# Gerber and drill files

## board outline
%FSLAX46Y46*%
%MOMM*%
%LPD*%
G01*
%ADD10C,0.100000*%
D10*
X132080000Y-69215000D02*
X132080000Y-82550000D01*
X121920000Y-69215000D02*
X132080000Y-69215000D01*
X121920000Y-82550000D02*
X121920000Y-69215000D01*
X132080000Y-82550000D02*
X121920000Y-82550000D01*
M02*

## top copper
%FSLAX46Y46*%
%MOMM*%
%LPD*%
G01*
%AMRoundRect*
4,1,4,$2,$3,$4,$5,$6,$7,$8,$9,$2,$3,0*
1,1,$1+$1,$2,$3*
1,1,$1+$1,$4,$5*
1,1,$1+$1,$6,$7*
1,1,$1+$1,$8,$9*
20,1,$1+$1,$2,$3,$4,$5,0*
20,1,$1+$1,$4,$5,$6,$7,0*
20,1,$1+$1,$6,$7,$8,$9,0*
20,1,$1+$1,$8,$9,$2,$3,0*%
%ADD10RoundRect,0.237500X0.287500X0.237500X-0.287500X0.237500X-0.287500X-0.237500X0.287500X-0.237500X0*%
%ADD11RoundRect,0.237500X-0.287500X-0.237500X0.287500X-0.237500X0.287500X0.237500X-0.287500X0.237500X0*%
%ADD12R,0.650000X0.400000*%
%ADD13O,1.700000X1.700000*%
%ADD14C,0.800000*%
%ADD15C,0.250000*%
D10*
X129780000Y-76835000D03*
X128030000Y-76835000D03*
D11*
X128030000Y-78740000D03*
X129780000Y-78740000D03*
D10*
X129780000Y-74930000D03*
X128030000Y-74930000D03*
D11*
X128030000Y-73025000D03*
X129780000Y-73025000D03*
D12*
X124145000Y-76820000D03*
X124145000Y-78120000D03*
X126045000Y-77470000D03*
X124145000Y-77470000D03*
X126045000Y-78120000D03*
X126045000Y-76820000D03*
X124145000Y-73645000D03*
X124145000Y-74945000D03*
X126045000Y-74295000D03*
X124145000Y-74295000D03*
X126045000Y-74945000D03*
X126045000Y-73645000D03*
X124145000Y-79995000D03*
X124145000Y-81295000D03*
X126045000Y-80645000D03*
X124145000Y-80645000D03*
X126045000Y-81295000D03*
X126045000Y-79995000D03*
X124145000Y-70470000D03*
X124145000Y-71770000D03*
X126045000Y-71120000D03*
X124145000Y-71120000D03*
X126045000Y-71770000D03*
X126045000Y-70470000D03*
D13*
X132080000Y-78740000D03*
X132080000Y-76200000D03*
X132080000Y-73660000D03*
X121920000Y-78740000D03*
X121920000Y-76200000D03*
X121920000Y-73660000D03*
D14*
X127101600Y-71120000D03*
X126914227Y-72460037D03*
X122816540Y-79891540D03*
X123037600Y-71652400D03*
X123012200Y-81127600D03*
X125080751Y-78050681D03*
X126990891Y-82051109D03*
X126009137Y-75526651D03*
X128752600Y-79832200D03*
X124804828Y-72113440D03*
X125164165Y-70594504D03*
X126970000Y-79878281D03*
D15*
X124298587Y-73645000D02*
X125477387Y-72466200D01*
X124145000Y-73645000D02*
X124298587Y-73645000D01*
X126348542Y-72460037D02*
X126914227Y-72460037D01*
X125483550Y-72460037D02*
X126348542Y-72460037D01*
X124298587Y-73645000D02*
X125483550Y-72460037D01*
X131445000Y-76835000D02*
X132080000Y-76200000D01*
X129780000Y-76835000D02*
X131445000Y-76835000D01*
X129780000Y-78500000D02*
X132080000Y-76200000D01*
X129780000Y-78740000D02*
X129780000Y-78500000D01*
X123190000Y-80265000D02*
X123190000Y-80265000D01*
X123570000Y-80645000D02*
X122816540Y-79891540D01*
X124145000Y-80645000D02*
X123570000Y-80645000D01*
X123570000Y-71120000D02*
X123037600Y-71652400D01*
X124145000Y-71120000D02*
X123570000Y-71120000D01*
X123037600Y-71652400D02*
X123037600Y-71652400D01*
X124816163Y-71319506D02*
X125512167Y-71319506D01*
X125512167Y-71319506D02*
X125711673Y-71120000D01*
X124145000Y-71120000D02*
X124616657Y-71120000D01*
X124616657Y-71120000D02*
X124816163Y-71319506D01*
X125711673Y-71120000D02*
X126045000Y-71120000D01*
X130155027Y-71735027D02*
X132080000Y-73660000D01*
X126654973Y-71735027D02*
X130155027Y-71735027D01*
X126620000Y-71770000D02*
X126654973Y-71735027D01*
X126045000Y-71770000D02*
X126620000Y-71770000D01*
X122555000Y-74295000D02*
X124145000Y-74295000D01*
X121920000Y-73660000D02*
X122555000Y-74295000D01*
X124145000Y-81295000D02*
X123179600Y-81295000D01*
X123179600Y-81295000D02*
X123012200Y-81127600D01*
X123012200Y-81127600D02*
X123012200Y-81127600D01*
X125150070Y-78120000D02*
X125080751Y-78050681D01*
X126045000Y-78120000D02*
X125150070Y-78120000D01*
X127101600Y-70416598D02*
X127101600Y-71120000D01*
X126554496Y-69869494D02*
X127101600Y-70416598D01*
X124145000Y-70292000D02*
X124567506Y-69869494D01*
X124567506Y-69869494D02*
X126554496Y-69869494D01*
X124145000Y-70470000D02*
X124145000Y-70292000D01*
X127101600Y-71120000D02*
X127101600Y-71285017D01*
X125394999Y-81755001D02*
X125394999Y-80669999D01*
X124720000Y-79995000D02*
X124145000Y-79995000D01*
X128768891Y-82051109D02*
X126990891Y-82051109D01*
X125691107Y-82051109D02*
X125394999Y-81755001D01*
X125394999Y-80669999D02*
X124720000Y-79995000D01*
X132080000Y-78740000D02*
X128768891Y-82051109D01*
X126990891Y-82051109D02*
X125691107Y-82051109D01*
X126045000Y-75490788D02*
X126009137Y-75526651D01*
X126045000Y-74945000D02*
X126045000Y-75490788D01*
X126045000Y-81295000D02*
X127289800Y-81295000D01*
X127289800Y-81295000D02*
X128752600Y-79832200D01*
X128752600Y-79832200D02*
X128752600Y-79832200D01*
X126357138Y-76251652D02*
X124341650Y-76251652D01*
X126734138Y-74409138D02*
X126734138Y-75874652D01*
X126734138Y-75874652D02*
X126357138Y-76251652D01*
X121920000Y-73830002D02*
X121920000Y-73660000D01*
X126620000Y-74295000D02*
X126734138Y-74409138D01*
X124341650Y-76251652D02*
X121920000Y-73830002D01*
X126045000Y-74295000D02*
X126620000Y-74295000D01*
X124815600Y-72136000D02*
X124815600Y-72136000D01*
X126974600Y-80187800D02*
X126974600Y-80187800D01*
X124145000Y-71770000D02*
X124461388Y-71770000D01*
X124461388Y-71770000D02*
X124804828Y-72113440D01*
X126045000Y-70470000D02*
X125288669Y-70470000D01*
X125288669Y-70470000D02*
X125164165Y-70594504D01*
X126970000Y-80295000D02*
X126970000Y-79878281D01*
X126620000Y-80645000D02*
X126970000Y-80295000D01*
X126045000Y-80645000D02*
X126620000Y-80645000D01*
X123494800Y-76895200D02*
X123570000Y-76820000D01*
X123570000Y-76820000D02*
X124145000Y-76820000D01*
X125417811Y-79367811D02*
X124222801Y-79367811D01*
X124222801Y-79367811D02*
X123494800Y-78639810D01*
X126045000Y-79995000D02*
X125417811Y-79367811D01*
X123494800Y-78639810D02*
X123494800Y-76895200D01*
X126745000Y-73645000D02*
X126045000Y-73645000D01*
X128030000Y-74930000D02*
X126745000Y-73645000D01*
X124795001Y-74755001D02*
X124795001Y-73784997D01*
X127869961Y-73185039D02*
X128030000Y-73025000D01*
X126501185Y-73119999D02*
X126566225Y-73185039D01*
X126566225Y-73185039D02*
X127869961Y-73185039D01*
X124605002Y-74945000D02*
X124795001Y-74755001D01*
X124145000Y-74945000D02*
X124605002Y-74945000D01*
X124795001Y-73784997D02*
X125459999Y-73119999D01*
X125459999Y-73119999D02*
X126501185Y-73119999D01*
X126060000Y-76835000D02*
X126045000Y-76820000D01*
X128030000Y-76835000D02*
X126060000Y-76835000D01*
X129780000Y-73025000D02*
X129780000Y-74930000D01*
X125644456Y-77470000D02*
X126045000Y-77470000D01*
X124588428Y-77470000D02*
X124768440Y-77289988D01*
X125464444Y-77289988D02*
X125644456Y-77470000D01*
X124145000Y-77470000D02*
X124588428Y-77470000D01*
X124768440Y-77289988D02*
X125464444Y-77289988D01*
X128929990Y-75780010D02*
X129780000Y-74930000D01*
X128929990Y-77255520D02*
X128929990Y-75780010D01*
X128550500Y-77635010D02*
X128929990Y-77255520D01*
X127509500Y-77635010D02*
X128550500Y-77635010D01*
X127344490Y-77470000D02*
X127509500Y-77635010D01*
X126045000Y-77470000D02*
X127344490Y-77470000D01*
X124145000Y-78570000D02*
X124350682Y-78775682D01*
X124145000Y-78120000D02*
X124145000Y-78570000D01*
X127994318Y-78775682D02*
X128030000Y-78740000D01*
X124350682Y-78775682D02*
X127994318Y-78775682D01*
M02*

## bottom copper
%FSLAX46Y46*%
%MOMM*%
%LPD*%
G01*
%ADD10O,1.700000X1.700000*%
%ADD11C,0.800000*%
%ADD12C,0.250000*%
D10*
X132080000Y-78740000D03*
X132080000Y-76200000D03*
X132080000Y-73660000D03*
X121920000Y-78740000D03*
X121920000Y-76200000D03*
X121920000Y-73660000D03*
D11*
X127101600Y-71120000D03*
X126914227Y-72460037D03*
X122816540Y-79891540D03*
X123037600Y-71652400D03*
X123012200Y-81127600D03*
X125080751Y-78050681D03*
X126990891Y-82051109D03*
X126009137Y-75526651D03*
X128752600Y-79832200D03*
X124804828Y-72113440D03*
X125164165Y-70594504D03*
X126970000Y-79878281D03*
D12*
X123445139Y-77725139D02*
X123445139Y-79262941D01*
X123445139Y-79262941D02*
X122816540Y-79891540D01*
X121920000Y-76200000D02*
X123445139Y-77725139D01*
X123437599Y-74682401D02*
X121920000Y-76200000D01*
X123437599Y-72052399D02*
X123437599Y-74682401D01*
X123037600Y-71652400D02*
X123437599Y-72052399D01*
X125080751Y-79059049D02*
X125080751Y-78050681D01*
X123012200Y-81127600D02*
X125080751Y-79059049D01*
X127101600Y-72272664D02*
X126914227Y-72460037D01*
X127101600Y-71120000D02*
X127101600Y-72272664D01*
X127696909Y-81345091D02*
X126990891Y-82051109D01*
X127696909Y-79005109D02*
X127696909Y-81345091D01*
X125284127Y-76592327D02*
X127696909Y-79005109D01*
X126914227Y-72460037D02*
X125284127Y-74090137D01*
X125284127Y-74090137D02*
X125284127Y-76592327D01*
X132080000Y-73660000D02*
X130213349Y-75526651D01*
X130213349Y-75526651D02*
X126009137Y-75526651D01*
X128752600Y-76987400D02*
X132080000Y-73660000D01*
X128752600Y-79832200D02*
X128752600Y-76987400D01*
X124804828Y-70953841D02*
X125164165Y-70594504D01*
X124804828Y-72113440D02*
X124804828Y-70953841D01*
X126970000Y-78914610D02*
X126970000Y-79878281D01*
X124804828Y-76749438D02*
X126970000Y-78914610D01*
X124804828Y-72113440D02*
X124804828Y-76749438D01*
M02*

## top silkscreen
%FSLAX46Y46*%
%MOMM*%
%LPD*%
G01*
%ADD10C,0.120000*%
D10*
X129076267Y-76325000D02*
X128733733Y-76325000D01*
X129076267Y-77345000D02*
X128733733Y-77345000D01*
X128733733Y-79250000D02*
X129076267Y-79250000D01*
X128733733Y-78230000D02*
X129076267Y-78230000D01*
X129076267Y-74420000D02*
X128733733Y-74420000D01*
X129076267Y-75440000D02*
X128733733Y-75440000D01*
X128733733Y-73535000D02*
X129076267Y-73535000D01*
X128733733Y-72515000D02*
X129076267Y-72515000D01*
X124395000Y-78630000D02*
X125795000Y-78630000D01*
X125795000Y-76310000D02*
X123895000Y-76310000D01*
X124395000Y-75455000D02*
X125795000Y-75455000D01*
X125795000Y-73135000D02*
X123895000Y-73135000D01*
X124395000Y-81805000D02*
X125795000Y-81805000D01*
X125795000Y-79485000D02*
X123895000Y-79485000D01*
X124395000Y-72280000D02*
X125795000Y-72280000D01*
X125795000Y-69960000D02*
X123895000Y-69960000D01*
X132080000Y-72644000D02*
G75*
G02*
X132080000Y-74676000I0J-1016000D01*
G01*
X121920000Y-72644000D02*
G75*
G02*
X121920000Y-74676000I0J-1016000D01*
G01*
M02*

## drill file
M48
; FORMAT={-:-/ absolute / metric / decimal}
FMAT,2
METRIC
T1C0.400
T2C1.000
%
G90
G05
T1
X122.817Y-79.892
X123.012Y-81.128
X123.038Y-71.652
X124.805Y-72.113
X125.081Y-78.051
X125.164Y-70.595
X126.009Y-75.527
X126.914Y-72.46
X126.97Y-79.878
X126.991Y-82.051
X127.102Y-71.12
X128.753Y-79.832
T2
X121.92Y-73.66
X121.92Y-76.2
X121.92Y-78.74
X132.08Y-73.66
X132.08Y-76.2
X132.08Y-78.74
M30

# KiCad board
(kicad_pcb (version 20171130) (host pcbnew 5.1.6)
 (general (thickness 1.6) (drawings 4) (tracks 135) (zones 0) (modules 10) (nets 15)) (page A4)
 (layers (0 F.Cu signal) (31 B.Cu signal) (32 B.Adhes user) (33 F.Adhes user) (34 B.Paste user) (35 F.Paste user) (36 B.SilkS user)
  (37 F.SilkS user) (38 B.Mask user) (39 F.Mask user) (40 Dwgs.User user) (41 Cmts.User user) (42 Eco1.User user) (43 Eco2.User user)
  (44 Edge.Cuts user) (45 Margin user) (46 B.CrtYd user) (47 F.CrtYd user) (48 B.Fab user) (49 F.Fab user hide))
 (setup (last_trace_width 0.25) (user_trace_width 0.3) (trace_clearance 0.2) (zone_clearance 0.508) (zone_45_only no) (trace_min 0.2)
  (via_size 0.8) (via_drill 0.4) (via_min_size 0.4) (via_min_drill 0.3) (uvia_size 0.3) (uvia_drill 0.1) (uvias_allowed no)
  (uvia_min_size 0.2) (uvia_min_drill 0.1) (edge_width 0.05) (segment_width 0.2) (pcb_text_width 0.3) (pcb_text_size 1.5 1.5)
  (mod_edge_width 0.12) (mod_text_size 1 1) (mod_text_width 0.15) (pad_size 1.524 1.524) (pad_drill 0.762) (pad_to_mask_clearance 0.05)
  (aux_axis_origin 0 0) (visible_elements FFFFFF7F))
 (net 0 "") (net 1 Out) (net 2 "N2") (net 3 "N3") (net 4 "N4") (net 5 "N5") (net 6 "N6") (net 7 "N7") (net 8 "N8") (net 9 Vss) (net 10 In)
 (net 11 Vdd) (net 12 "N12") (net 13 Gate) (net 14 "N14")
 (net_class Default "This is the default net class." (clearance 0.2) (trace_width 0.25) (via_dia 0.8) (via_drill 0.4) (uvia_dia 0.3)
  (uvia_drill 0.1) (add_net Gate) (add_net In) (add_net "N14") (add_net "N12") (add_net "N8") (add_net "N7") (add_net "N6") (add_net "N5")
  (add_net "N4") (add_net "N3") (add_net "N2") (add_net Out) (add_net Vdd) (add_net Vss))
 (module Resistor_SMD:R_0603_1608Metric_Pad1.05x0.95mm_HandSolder (layer F.Cu) (at 128.905 76.835 180)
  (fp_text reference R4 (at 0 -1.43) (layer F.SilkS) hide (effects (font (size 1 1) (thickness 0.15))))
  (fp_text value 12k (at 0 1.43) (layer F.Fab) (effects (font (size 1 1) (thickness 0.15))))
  (fp_line (start -0.171267 0.51) (end 0.171267 0.51) (layer F.SilkS) (width 0.12))
  (fp_line (start -0.171267 -0.51) (end 0.171267 -0.51) (layer F.SilkS) (width 0.12))
  (pad 1 smd roundrect (at -0.875 0 180) (size 1.05 0.95) (layers F.Cu F.Paste F.Mask) (roundrect_rratio 0.25) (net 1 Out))
  (pad 2 smd roundrect (at 0.875 0 180) (size 1.05 0.95) (layers F.Cu F.Paste F.Mask) (roundrect_rratio 0.25) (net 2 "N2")))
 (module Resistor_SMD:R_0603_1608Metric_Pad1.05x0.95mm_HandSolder (layer F.Cu) (at 128.905 78.74)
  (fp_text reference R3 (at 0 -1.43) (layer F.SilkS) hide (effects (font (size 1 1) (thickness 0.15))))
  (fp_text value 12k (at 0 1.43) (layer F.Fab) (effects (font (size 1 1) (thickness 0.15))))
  (fp_line (start -0.171267 0.51) (end 0.171267 0.51) (layer F.SilkS) (width 0.12))
  (fp_line (start -0.171267 -0.51) (end 0.171267 -0.51) (layer F.SilkS) (width 0.12))
  (pad 1 smd roundrect (at -0.875 0) (size 1.05 0.95) (layers F.Cu F.Paste F.Mask) (roundrect_rratio 0.25) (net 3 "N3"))
  (pad 2 smd roundrect (at 0.875 0) (size 1.05 0.95) (layers F.Cu F.Paste F.Mask) (roundrect_rratio 0.25) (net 1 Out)))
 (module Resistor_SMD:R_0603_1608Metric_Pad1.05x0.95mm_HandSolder (layer F.Cu) (at 128.905 74.93 180)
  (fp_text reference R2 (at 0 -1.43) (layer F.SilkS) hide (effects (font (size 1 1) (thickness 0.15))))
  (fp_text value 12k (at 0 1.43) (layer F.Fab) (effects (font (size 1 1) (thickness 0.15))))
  (fp_line (start -0.171267 0.51) (end 0.171267 0.51) (layer F.SilkS) (width 0.12))
  (fp_line (start -0.171267 -0.51) (end 0.171267 -0.51) (layer F.SilkS) (width 0.12))
  (pad 1 smd roundrect (at -0.875 0 180) (size 1.05 0.95) (layers F.Cu F.Paste F.Mask) (roundrect_rratio 0.25) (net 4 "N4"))
  (pad 2 smd roundrect (at 0.875 0 180) (size 1.05 0.95) (layers F.Cu F.Paste F.Mask) (roundrect_rratio 0.25) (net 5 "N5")))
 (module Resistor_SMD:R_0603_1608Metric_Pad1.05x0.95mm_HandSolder (layer F.Cu) (at 128.905 73.025)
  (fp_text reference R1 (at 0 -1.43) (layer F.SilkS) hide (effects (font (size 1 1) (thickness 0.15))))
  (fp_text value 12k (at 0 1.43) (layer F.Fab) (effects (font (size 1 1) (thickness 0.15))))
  (fp_line (start -0.171267 0.51) (end 0.171267 0.51) (layer F.SilkS) (width 0.12))
  (fp_line (start -0.171267 -0.51) (end 0.171267 -0.51) (layer F.SilkS) (width 0.12))
  (pad 1 smd roundrect (at -0.875 0) (size 1.05 0.95) (layers F.Cu F.Paste F.Mask) (roundrect_rratio 0.25) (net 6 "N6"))
  (pad 2 smd roundrect (at 0.875 0) (size 1.05 0.95) (layers F.Cu F.Paste F.Mask) (roundrect_rratio 0.25) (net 4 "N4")))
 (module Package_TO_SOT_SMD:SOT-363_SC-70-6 (layer F.Cu) (at 125.095 77.47)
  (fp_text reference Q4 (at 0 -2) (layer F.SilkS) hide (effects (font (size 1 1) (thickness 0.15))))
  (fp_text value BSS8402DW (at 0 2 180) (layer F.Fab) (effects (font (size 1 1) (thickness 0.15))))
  (fp_line (start -0.7 1.16) (end 0.7 1.16) (layer F.SilkS) (width 0.12))
  (fp_line (start 0.7 -1.16) (end -1.2 -1.16) (layer F.SilkS) (width 0.12))
  (pad 1 smd rect (at -0.95 -0.65) (size 0.65 0.4) (layers F.Cu F.Paste F.Mask) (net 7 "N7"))
  (pad 3 smd rect (at -0.95 0.65) (size 0.65 0.4) (layers F.Cu F.Paste F.Mask) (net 3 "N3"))
  (pad 5 smd rect (at 0.95 0) (size 0.65 0.4) (layers F.Cu F.Paste F.Mask) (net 4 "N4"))
  (pad 2 smd rect (at -0.95 0) (size 0.65 0.4) (layers F.Cu F.Paste F.Mask) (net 4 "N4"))
  (pad 4 smd rect (at 0.95 0.65) (size 0.65 0.4) (layers F.Cu F.Paste F.Mask) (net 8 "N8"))
  (pad 6 smd rect (at 0.95 -0.65) (size 0.65 0.4) (layers F.Cu F.Paste F.Mask) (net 2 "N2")))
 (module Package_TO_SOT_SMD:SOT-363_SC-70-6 (layer F.Cu) (at 125.095 74.295)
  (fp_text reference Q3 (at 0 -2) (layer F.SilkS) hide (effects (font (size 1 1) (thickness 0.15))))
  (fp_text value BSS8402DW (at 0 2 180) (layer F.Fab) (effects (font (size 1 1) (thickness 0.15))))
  (fp_line (start -0.7 1.16) (end 0.7 1.16) (layer F.SilkS) (width 0.12))
  (fp_line (start 0.7 -1.16) (end -1.2 -1.16) (layer F.SilkS) (width 0.12))
  (pad 1 smd rect (at -0.95 -0.65) (size 0.65 0.4) (layers F.Cu F.Paste F.Mask) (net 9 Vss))
  (pad 3 smd rect (at -0.95 0.65) (size 0.65 0.4) (layers F.Cu F.Paste F.Mask) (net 6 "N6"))
  (pad 5 smd rect (at 0.95 0) (size 0.65 0.4) (layers F.Cu F.Paste F.Mask) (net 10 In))
  (pad 2 smd rect (at -0.95 0) (size 0.65 0.4) (layers F.Cu F.Paste F.Mask) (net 10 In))
  (pad 4 smd rect (at 0.95 0.65) (size 0.65 0.4) (layers F.Cu F.Paste F.Mask) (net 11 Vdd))
  (pad 6 smd rect (at 0.95 -0.65) (size 0.65 0.4) (layers F.Cu F.Paste F.Mask) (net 5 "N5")))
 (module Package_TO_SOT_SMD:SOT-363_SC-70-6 (layer F.Cu) (at 125.095 80.645)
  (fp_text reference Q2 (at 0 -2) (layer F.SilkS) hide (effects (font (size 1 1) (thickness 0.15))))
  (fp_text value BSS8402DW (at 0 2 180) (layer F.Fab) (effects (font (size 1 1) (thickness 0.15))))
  (fp_line (start -0.7 1.16) (end 0.7 1.16) (layer F.SilkS) (width 0.12))
  (fp_line (start 0.7 -1.16) (end -1.2 -1.16) (layer F.SilkS) (width 0.12))
  (pad 1 smd rect (at -0.95 -0.65) (size 0.65 0.4) (layers F.Cu F.Paste F.Mask) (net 9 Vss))
  (pad 3 smd rect (at -0.95 0.65) (size 0.65 0.4) (layers F.Cu F.Paste F.Mask) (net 8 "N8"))
  (pad 5 smd rect (at 0.95 0) (size 0.65 0.4) (layers F.Cu F.Paste F.Mask) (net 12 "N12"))
  (pad 2 smd rect (at -0.95 0) (size 0.65 0.4) (layers F.Cu F.Paste F.Mask) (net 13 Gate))
  (pad 4 smd rect (at 0.95 0.65) (size 0.65 0.4) (layers F.Cu F.Paste F.Mask) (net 11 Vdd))
  (pad 6 smd rect (at 0.95 -0.65) (size 0.65 0.4) (layers F.Cu F.Paste F.Mask) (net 7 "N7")))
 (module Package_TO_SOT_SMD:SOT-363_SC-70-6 (layer F.Cu) (at 125.095 71.12)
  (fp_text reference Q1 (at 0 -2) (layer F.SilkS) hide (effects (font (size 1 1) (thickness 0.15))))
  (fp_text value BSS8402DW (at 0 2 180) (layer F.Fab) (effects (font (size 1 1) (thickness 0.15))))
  (fp_line (start -0.7 1.16) (end 0.7 1.16) (layer F.SilkS) (width 0.12))
  (fp_line (start 0.7 -1.16) (end -1.2 -1.16) (layer F.SilkS) (width 0.12))
  (pad 1 smd rect (at -0.95 -0.65) (size 0.65 0.4) (layers F.Cu F.Paste F.Mask) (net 9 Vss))
  (pad 3 smd rect (at -0.95 0.65) (size 0.65 0.4) (layers F.Cu F.Paste F.Mask) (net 12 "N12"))
  (pad 5 smd rect (at 0.95 0) (size 0.65 0.4) (layers F.Cu F.Paste F.Mask) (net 13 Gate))
  (pad 2 smd rect (at -0.95 0) (size 0.65 0.4) (layers F.Cu F.Paste F.Mask) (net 13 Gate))
  (pad 4 smd rect (at 0.95 0.65) (size 0.65 0.4) (layers F.Cu F.Paste F.Mask) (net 11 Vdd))
  (pad 6 smd rect (at 0.95 -0.65) (size 0.65 0.4) (layers F.Cu F.Paste F.Mask) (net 12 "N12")))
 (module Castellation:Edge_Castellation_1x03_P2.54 (layer F.Cu) (at 132.08 73.66)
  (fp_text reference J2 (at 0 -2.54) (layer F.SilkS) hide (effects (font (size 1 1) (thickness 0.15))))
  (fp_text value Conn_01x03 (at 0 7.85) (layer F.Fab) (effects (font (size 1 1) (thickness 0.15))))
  (fp_arc (start 0 0) (end 0 1.016) (angle -180) (layer F.SilkS) (width 0.12))
  (pad 3 thru_hole oval (at 0 5.08) (size 1.7 1.7) (drill 1) (layers *.Cu *.Mask) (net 9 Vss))
  (pad 2 thru_hole oval (at 0 2.54) (size 1.7 1.7) (drill 1) (layers *.Cu *.Mask) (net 1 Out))
  (pad 1 thru_hole oval (at 0 0) (size 1.7 1.7) (drill 1) (layers *.Cu *.Mask) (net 11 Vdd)))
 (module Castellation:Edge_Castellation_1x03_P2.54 (layer F.Cu) (at 121.92 73.66)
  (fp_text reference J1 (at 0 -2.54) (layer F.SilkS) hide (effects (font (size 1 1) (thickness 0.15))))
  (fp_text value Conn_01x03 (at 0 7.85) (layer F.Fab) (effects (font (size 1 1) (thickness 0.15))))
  (fp_arc (start 0 0) (end 0 1.016) (angle -180) (layer F.SilkS) (width 0.12))
  (pad 3 thru_hole oval (at 0 5.08) (size 1.7 1.7) (drill 1) (layers *.Cu *.Mask) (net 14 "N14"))
  (pad 2 thru_hole oval (at 0 2.54) (size 1.7 1.7) (drill 1) (layers *.Cu *.Mask) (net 13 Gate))
  (pad 1 thru_hole oval (at 0 0) (size 1.7 1.7) (drill 1) (layers *.Cu *.Mask) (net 10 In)))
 (gr_line (start 132.08 69.215) (end 132.08 82.55) (layer Edge.Cuts) (width 0.1))
 (gr_line (start 121.92 69.215) (end 132.08 69.215) (layer Edge.Cuts) (width 0.1))
 (gr_line (start 121.92 82.55) (end 121.92 69.215) (layer Edge.Cuts) (width 0.1))
 (gr_line (start 132.08 82.55) (end 121.92 82.55) (layer Edge.Cuts) (width 0.1))
 (via (at 127.1016 71.12) (size 0.8) (drill 0.4) (layers F.Cu B.Cu) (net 9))
 (segment (start 124.298587 73.645) (end 125.477387 72.4662) (width 0.25) (layer F.Cu) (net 9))
 (segment (start 124.145 73.645) (end 124.298587 73.645) (width 0.25) (layer F.Cu) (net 9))
 (segment (start 126.348542 72.460037) (end 126.914227 72.460037) (width 0.25) (layer F.Cu) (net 9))
 (segment (start 125.48355 72.460037) (end 126.348542 72.460037) (width 0.25) (layer F.Cu) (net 9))
 (via (at 126.914227 72.460037) (size 0.8) (drill 0.4) (layers F.Cu B.Cu) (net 9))
 (segment (start 124.298587 73.645) (end 125.48355 72.460037) (width 0.25) (layer F.Cu) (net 9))
 (segment (start 131.445 76.835) (end 132.08 76.2) (width 0.25) (layer F.Cu) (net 1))
 (segment (start 129.78 76.835) (end 131.445 76.835) (width 0.25) (layer F.Cu) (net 1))
 (segment (start 129.78 78.5) (end 132.08 76.2) (width 0.25) (layer F.Cu) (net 1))
 (segment (start 129.78 78.74) (end 129.78 78.5) (width 0.25) (layer F.Cu) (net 1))
 (segment (start 123.19 80.265) (end 123.19 80.265) (width 0.25) (layer F.Cu) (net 13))
 (segment (start 123.445139 77.725139) (end 123.445139 79.262941) (width 0.25) (layer B.Cu) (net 13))
 (segment (start 123.57 80.645) (end 122.81654 79.89154) (width 0.25) (layer F.Cu) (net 13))
 (segment (start 124.145 80.645) (end 123.57 80.645) (width 0.25) (layer F.Cu) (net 13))
 (segment (start 123.445139 79.262941) (end 122.81654 79.89154) (width 0.25) (layer B.Cu) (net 13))
 (via (at 122.81654 79.89154) (size 0.8) (drill 0.4) (layers F.Cu B.Cu) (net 13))
 (segment (start 121.92 76.2) (end 123.445139 77.725139) (width 0.25) (layer B.Cu) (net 13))
 (segment (start 123.57 71.12) (end 123.0376 71.6524) (width 0.25) (layer F.Cu) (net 13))
 (segment (start 124.145 71.12) (end 123.57 71.12) (width 0.25) (layer F.Cu) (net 13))
 (segment (start 123.0376 71.6524) (end 123.0376 71.6524) (width 0.25) (layer F.Cu) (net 13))
 (via (at 123.0376 71.6524) (size 0.8) (drill 0.4) (layers F.Cu B.Cu) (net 13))
 (segment (start 123.437599 74.682401) (end 121.92 76.2) (width 0.25) (layer B.Cu) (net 13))
 (segment (start 123.437599 72.052399) (end 123.437599 74.682401) (width 0.25) (layer B.Cu) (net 13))
 (segment (start 123.0376 71.6524) (end 123.437599 72.052399) (width 0.25) (layer B.Cu) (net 13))
 (segment (start 124.816163 71.319506) (end 125.512167 71.319506) (width 0.25) (layer F.Cu) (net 13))
 (segment (start 125.512167 71.319506) (end 125.711673 71.12) (width 0.25) (layer F.Cu) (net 13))
 (segment (start 124.145 71.12) (end 124.616657 71.12) (width 0.25) (layer F.Cu) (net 13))
 (segment (start 124.616657 71.12) (end 124.816163 71.319506) (width 0.25) (layer F.Cu) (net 13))
 (segment (start 125.711673 71.12) (end 126.045 71.12) (width 0.25) (layer F.Cu) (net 13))
 (segment (start 130.155027 71.735027) (end 132.08 73.66) (width 0.25) (layer F.Cu) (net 11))
 (segment (start 126.654973 71.735027) (end 130.155027 71.735027) (width 0.25) (layer F.Cu) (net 11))
 (segment (start 126.62 71.77) (end 126.654973 71.735027) (width 0.25) (layer F.Cu) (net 11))
 (segment (start 126.045 71.77) (end 126.62 71.77) (width 0.25) (layer F.Cu) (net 11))
 (segment (start 122.555 74.295) (end 124.145 74.295) (width 0.25) (layer F.Cu) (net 10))
 (segment (start 121.92 73.66) (end 122.555 74.295) (width 0.25) (layer F.Cu) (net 10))
 (segment (start 124.145 81.295) (end 123.1796 81.295) (width 0.25) (layer F.Cu) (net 8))
 (segment (start 123.1796 81.295) (end 123.0122 81.1276) (width 0.25) (layer F.Cu) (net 8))
 (segment (start 123.0122 81.1276) (end 123.0122 81.1276) (width 0.25) (layer F.Cu) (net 8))
 (via (at 123.0122 81.1276) (size 0.8) (drill 0.4) (layers F.Cu B.Cu) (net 8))
 (segment (start 125.15007 78.12) (end 125.080751 78.050681) (width 0.25) (layer F.Cu) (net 8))
 (via (at 125.080751 78.050681) (size 0.8) (drill 0.4) (layers F.Cu B.Cu) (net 8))
 (segment (start 125.080751 79.059049) (end 125.080751 78.050681) (width 0.25) (layer B.Cu) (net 8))
 (segment (start 123.0122 81.1276) (end 125.080751 79.059049) (width 0.25) (layer B.Cu) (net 8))
 (segment (start 126.045 78.12) (end 125.15007 78.12) (width 0.25) (layer F.Cu) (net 8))
 (segment (start 127.1016 70.416598) (end 127.1016 71.12) (width 0.25) (layer F.Cu) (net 9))
 (segment (start 126.554496 69.869494) (end 127.1016 70.416598) (width 0.25) (layer F.Cu) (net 9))
 (segment (start 124.145 70.292) (end 124.567506 69.869494) (width 0.25) (layer F.Cu) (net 9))
 (segment (start 124.567506 69.869494) (end 126.554496 69.869494) (width 0.25) (layer F.Cu) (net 9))
 (segment (start 124.145 70.47) (end 124.145 70.292) (width 0.25) (layer F.Cu) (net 9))
 (segment (start 127.1016 71.12) (end 127.1016 71.285017) (width 0.25) (layer F.Cu) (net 9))
 (segment (start 127.1016 72.272664) (end 126.914227 72.460037) (width 0.25) (layer B.Cu) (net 9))
 (segment (start 127.1016 71.12) (end 127.1016 72.272664) (width 0.25) (layer B.Cu) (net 9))
 (segment (start 125.394999 81.755001) (end 125.394999 80.669999) (width 0.25) (layer F.Cu) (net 9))
 (segment (start 124.72 79.995) (end 124.145 79.995) (width 0.25) (layer F.Cu) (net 9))
 (segment (start 128.768891 82.051109) (end 126.990891 82.051109) (width 0.25) (layer F.Cu) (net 9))
 (segment (start 125.691107 82.051109) (end 125.394999 81.755001) (width 0.25) (layer F.Cu) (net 9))
 (segment (start 125.394999 80.669999) (end 124.72 79.995) (width 0.25) (layer F.Cu) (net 9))
 (segment (start 132.08 78.74) (end 128.768891 82.051109) (width 0.25) (layer F.Cu) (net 9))
 (segment (start 126.990891 82.051109) (end 125.691107 82.051109) (width 0.25) (layer F.Cu) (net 9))
 (via (at 126.990891 82.051109) (size 0.8) (drill 0.4) (layers F.Cu B.Cu) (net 9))
 (segment (start 127.696909 81.345091) (end 126.990891 82.051109) (width 0.25) (layer B.Cu) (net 9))
 (segment (start 127.696909 79.005109) (end 127.696909 81.345091) (width 0.25) (layer B.Cu) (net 9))
 (segment (start 125.284127 76.592327) (end 127.696909 79.005109) (width 0.25) (layer B.Cu) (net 9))
 (segment (start 126.914227 72.460037) (end 125.284127 74.090137) (width 0.25) (layer B.Cu) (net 9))
 (segment (start 125.284127 74.090137) (end 125.284127 76.592327) (width 0.25) (layer B.Cu) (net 9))
 (via (at 126.009137 75.526651) (size 0.8) (drill 0.4) (layers F.Cu B.Cu) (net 11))
 (segment (start 132.08 73.66) (end 130.213349 75.526651) (width 0.25) (layer B.Cu) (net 11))
 (segment (start 130.213349 75.526651) (end 126.009137 75.526651) (width 0.25) (layer B.Cu) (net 11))
 (segment (start 126.045 75.490788) (end 126.009137 75.526651) (width 0.25) (layer F.Cu) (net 11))
 (segment (start 126.045 74.945) (end 126.045 75.490788) (width 0.25) (layer F.Cu) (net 11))
 (segment (start 126.045 81.295) (end 127.2898 81.295) (width 0.25) (layer F.Cu) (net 11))
 (segment (start 127.2898 81.295) (end 128.7526 79.8322) (width 0.25) (layer F.Cu) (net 11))
 (segment (start 128.7526 79.8322) (end 128.7526 79.8322) (width 0.25) (layer F.Cu) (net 11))
 (via (at 128.7526 79.8322) (size 0.8) (drill 0.4) (layers F.Cu B.Cu) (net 11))
 (segment (start 128.7526 76.9874) (end 132.08 73.66) (width 0.25) (layer B.Cu) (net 11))
 (segment (start 128.7526 79.8322) (end 128.7526 76.9874) (width 0.25) (layer B.Cu) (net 11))
 (segment (start 126.357138 76.251652) (end 124.34165 76.251652) (width 0.25) (layer F.Cu) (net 10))
 (segment (start 126.734138 74.409138) (end 126.734138 75.874652) (width 0.25) (layer F.Cu) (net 10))
 (segment (start 126.734138 75.874652) (end 126.357138 76.251652) (width 0.25) (layer F.Cu) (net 10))
 (segment (start 121.92 73.830002) (end 121.92 73.66) (width 0.25) (layer F.Cu) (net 10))
 (segment (start 126.62 74.295) (end 126.734138 74.409138) (width 0.25) (layer F.Cu) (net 10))
 (segment (start 124.34165 76.251652) (end 121.92 73.830002) (width 0.25) (layer F.Cu) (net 10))
 (segment (start 126.045 74.295) (end 126.62 74.295) (width 0.25) (layer F.Cu) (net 10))
 (segment (start 124.8156 72.136) (end 124.8156 72.136) (width 0.25) (layer F.Cu) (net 12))
 (segment (start 126.9746 80.1878) (end 126.9746 80.1878) (width 0.25) (layer F.Cu) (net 12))
 (via (at 124.804828 72.11344) (size 0.8) (drill 0.4) (layers F.Cu B.Cu) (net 12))
 (segment (start 124.145 71.77) (end 124.461388 71.77) (width 0.25) (layer F.Cu) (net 12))
 (segment (start 124.461388 71.77) (end 124.804828 72.11344) (width 0.25) (layer F.Cu) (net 12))
 (segment (start 126.045 70.47) (end 125.288669 70.47) (width 0.25) (layer F.Cu) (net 12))
 (segment (start 124.804828 70.953841) (end 125.164165 70.594504) (width 0.25) (layer B.Cu) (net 12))
 (segment (start 124.804828 72.11344) (end 124.804828 70.953841) (width 0.25) (layer B.Cu) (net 12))
 (segment (start 125.288669 70.47) (end 125.164165 70.594504) (width 0.25) (layer F.Cu) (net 12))
 (via (at 125.164165 70.594504) (size 0.8) (drill 0.4) (layers F.Cu B.Cu) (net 12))
 (segment (start 126.97 78.91461) (end 126.97 79.878281) (width 0.25) (layer B.Cu) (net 12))
 (via (at 126.97 79.878281) (size 0.8) (drill 0.4) (layers F.Cu B.Cu) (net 12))
 (segment (start 126.97 80.295) (end 126.97 79.878281) (width 0.25) (layer F.Cu) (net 12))
 (segment (start 124.804828 76.749438) (end 126.97 78.91461) (width 0.25) (layer B.Cu) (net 12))
 (segment (start 124.804828 72.11344) (end 124.804828 76.749438) (width 0.25) (layer B.Cu) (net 12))
 (segment (start 126.62 80.645) (end 126.97 80.295) (width 0.25) (layer F.Cu) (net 12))
 (segment (start 126.045 80.645) (end 126.62 80.645) (width 0.25) (layer F.Cu) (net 12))
 (segment (start 123.4948 76.8952) (end 123.57 76.82) (width 0.25) (layer F.Cu) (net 7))
 (segment (start 123.57 76.82) (end 124.145 76.82) (width 0.25) (layer F.Cu) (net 7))
 (segment (start 125.417811 79.367811) (end 124.222801 79.367811) (width 0.25) (layer F.Cu) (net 7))
 (segment (start 124.222801 79.367811) (end 123.4948 78.63981) (width 0.25) (layer F.Cu) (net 7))
 (segment (start 126.045 79.995) (end 125.417811 79.367811) (width 0.25) (layer F.Cu) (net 7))
 (segment (start 123.4948 78.63981) (end 123.4948 76.8952) (width 0.25) (layer F.Cu) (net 7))
 (segment (start 126.745 73.645) (end 126.045 73.645) (width 0.25) (layer F.Cu) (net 5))
 (segment (start 128.03 74.93) (end 126.745 73.645) (width 0.25) (layer F.Cu) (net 5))
 (segment (start 124.795001 74.755001) (end 124.795001 73.784997) (width 0.25) (layer F.Cu) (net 6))
 (segment (start 127.869961 73.185039) (end 128.03 73.025) (width 0.25) (layer F.Cu) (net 6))
 (segment (start 126.501185 73.119999) (end 126.566225 73.185039) (width 0.25) (layer F.Cu) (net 6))
 (segment (start 126.566225 73.185039) (end 127.869961 73.185039) (width 0.25) (layer F.Cu) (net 6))
 (segment (start 124.605002 74.945) (end 124.795001 74.755001) (width 0.25) (layer F.Cu) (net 6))
 (segment (start 124.145 74.945) (end 124.605002 74.945) (width 0.25) (layer F.Cu) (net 6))
 (segment (start 124.795001 73.784997) (end 125.459999 73.119999) (width 0.25) (layer F.Cu) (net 6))
 (segment (start 125.459999 73.119999) (end 126.501185 73.119999) (width 0.25) (layer F.Cu) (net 6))
 (segment (start 126.06 76.835) (end 126.045 76.82) (width 0.25) (layer F.Cu) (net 2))
 (segment (start 128.03 76.835) (end 126.06 76.835) (width 0.25) (layer F.Cu) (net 2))
 (segment (start 129.78 73.025) (end 129.78 74.93) (width 0.25) (layer F.Cu) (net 4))
 (segment (start 125.644456 77.47) (end 126.045 77.47) (width 0.25) (layer F.Cu) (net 4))
 (segment (start 124.588428 77.47) (end 124.76844 77.289988) (width 0.25) (layer F.Cu) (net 4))
 (segment (start 125.464444 77.289988) (end 125.644456 77.47) (width 0.25) (layer F.Cu) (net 4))
 (segment (start 124.145 77.47) (end 124.588428 77.47) (width 0.25) (layer F.Cu) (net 4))
 (segment (start 124.76844 77.289988) (end 125.464444 77.289988) (width 0.25) (layer F.Cu) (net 4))
 (segment (start 128.92999 75.78001) (end 129.78 74.93) (width 0.25) (layer F.Cu) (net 4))
 (segment (start 128.92999 77.25552) (end 128.92999 75.78001) (width 0.25) (layer F.Cu) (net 4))
 (segment (start 128.5505 77.63501) (end 128.92999 77.25552) (width 0.25) (layer F.Cu) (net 4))
 (segment (start 127.5095 77.63501) (end 128.5505 77.63501) (width 0.25) (layer F.Cu) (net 4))
 (segment (start 127.34449 77.47) (end 127.5095 77.63501) (width 0.25) (layer F.Cu) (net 4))
 (segment (start 126.045 77.47) (end 127.34449 77.47) (width 0.25) (layer F.Cu) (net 4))
 (segment (start 124.145 78.57) (end 124.350682 78.775682) (width 0.25) (layer F.Cu) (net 3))
 (segment (start 124.145 78.12) (end 124.145 78.57) (width 0.25) (layer F.Cu) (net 3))
 (segment (start 127.994318 78.775682) (end 128.03 78.74) (width 0.25) (layer F.Cu) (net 3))
 (segment (start 124.350682 78.775682) (end 127.994318 78.775682) (width 0.25) (layer F.Cu) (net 3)))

